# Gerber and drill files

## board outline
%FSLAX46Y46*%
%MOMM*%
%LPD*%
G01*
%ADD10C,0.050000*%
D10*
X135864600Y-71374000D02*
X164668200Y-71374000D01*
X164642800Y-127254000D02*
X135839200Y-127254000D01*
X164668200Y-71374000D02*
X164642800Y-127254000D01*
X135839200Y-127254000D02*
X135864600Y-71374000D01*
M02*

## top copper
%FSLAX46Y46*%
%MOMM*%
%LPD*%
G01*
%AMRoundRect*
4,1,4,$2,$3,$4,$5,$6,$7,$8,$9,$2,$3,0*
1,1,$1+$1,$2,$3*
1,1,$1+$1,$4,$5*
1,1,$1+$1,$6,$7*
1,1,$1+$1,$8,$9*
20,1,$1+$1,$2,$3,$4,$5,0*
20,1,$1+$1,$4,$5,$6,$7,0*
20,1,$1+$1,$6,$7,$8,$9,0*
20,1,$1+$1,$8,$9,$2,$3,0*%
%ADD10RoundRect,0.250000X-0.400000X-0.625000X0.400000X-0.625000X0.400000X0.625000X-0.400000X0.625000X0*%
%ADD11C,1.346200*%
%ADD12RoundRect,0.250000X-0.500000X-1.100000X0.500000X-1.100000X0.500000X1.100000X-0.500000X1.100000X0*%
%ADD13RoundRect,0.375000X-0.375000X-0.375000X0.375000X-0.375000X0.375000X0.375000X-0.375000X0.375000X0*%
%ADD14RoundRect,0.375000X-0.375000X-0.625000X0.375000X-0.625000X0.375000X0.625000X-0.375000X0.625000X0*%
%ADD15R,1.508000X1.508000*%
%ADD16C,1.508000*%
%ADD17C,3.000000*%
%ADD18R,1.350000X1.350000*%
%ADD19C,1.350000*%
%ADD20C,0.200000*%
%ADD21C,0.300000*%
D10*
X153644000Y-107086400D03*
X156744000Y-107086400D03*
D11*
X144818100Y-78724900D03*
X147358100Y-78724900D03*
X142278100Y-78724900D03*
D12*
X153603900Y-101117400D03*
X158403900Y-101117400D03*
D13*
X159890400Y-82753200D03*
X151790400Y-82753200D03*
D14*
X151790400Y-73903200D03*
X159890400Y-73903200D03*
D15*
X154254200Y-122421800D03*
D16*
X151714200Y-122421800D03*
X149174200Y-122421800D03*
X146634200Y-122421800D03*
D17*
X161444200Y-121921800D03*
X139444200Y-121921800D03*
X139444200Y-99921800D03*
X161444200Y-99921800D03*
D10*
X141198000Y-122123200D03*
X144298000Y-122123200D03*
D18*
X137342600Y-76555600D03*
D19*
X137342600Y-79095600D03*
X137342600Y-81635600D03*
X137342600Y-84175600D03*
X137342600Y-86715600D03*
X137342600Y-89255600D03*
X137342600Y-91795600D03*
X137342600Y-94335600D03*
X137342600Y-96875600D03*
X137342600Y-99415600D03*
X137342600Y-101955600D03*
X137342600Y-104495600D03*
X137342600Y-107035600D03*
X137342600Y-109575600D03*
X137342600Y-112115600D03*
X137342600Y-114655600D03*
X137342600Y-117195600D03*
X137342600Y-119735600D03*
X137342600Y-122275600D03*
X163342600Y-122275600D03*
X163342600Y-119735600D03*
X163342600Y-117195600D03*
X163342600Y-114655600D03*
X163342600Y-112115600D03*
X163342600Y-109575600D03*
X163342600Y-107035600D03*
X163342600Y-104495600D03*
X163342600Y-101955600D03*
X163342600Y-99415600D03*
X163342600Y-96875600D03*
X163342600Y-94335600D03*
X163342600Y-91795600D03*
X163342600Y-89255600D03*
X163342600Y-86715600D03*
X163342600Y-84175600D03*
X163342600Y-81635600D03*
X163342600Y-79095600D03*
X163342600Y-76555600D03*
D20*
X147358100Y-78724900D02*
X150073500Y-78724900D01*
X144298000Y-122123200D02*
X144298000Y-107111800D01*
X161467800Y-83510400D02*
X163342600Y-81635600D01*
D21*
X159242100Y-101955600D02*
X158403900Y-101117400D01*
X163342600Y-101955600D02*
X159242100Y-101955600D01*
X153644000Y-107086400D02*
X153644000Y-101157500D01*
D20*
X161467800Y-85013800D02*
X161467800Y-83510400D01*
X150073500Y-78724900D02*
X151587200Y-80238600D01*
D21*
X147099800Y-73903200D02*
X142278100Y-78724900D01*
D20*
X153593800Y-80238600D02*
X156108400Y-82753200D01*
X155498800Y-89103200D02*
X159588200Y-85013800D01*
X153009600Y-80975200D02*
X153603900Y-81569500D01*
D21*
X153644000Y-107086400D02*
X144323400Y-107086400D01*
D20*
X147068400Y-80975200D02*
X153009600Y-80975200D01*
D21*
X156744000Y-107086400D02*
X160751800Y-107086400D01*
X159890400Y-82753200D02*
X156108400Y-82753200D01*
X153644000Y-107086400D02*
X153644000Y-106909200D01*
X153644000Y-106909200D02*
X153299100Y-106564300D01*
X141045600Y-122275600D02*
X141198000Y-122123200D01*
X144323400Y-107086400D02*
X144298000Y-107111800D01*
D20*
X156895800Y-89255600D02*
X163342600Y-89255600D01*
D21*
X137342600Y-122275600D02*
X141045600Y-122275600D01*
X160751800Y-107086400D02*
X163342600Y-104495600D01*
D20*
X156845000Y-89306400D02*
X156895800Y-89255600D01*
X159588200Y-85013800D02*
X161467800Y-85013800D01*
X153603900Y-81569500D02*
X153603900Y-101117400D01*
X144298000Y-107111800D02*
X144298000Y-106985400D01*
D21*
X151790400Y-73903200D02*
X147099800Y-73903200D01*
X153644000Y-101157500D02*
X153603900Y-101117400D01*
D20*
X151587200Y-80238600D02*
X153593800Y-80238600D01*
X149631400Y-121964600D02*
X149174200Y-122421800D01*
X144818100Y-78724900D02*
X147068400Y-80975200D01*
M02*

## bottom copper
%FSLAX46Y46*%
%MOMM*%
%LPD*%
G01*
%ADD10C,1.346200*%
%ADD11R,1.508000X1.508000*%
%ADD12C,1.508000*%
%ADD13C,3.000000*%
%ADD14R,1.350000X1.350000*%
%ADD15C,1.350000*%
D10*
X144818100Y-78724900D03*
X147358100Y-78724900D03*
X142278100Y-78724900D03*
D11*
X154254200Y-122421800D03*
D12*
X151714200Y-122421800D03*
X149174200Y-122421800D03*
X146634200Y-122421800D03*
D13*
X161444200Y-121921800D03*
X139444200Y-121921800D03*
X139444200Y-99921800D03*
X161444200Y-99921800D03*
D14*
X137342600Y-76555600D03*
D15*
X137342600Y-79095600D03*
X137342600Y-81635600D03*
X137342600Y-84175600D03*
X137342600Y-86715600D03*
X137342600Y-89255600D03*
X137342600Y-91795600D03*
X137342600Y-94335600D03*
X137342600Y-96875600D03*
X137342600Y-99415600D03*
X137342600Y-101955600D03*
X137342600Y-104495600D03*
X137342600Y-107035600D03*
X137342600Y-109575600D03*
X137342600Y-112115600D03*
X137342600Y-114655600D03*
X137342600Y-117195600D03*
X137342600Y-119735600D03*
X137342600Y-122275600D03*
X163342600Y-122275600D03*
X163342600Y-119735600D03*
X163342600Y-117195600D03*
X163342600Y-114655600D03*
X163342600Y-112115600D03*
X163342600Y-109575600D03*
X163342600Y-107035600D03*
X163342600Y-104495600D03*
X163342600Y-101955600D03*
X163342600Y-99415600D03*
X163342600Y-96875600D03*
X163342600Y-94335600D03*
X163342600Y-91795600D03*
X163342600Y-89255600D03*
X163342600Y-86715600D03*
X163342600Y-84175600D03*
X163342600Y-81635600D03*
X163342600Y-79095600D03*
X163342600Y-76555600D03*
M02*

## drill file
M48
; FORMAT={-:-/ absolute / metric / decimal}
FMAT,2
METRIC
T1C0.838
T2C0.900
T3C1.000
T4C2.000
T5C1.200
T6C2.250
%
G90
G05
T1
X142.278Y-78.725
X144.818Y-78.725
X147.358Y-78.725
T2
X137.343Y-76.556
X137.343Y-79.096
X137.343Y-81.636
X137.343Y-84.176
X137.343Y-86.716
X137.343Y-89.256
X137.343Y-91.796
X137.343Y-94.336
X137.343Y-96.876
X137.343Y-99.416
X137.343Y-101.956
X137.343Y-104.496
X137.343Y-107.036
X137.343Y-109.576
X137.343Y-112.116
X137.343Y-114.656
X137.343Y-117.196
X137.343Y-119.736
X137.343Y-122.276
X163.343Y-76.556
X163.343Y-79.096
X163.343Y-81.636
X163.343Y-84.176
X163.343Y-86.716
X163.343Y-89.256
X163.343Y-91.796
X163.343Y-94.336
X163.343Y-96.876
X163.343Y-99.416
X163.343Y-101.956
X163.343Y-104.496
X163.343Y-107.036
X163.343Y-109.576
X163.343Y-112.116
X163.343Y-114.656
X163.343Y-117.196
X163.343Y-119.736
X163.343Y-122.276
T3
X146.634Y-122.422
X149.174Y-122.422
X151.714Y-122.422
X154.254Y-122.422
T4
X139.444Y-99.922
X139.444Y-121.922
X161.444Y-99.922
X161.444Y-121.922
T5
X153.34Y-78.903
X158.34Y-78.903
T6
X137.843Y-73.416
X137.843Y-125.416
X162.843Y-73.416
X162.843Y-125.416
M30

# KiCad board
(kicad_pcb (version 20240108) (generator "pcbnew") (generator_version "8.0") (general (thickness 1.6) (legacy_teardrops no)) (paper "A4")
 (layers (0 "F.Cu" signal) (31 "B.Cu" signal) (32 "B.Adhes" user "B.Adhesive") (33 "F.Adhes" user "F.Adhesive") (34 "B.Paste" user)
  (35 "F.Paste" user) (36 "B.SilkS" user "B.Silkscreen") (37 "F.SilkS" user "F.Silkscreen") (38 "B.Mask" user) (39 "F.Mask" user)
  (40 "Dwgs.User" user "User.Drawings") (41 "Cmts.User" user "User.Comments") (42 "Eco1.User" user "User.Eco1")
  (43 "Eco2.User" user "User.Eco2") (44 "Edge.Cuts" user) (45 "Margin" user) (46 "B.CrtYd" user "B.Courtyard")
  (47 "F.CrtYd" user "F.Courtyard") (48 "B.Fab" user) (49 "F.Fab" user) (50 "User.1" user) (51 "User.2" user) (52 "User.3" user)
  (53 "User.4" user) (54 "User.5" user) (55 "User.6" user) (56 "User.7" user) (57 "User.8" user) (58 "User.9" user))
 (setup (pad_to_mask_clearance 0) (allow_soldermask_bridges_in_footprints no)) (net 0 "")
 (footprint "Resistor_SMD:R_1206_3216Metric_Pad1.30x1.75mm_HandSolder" (layer "F.Cu") (at 155.194 107.0864)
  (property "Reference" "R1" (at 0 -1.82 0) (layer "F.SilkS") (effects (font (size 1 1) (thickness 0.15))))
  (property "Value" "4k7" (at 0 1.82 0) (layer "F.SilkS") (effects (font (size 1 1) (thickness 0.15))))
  (pad "1" smd roundrect (at -1.55 0) (size 1.3 1.75) (layers "F.Cu" "F.Paste" "F.Mask") (roundrect_rratio 0.192308))
  (pad "2" smd roundrect (at 1.55 0) (size 1.3 1.75) (layers "F.Cu" "F.Paste" "F.Mask") (roundrect_rratio 0.192308)))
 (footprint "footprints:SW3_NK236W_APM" (layer "F.Cu") (at 144.8181 78.7249 180)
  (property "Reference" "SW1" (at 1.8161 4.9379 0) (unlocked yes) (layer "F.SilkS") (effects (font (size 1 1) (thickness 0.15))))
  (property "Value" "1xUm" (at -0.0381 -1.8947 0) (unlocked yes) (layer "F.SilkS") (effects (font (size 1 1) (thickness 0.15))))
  (pad "1" thru_hole circle (at 0 0 180) (size 1.3462 1.3462) (drill 0.8382) (layers "*.Cu" "*.Mask") (remove_unused_layers no))
  (pad "2" thru_hole circle (at -2.54 0 180) (size 1.3462 1.3462) (drill 0.8382) (layers "*.Cu" "*.Mask") (remove_unused_layers no))
  (pad "3" thru_hole circle (at 2.54 0 180) (size 1.3462 1.3462) (drill 0.8382) (layers "*.Cu" "*.Mask") (remove_unused_layers no)))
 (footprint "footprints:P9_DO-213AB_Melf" (layer "F.Cu") (at 153.6039 101.1174)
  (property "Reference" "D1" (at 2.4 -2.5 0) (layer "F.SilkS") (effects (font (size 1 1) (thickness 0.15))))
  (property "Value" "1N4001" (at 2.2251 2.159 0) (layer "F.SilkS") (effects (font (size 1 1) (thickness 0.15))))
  (pad "1" smd roundrect (at 0 0) (size 1.5 2.7) (layers "F.Cu" "F.Paste" "F.Mask") (roundrect_rratio 0.1666666667))
  (pad "2" smd roundrect (at 4.8 0) (size 1.5 2.7) (layers "F.Cu" "F.Paste" "F.Mask") (roundrect_rratio 0.1666666667)))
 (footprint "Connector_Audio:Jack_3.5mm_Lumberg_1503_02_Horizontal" (layer "F.Cu") (at 155.8404 76.4032)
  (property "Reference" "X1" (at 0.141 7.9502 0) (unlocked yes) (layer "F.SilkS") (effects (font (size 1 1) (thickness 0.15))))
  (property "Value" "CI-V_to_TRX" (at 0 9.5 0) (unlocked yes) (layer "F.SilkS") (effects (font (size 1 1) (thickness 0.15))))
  (pad "" np_thru_hole circle (at -2.5 2.5) (size 1.2 1.2) (drill 1.2) (layers "F&B.Cu" "*.Mask"))
  (pad "" np_thru_hole circle (at 2.5 2.5) (size 1.2 1.2) (drill 1.2) (layers "F&B.Cu" "*.Mask"))
  (pad "R" smd roundrect (at 4.05 6.35) (size 1.5 1.5) (layers "F.Cu" "F.Paste" "F.Mask") (roundrect_rratio 0.25))
  (pad "S" smd roundrect (at -4.05 6.35) (size 1.5 1.5) (layers "F.Cu" "F.Paste" "F.Mask") (roundrect_rratio 0.25))
  (pad "T" smd roundrect (at -4.05 -2.5) (size 1.5 2) (layers "F.Cu" "F.Paste" "F.Mask") (roundrect_rratio 0.25))
  (pad "T" smd roundrect (at 4.05 -2.5) (size 1.5 2) (layers "F.Cu" "F.Paste" "F.Mask") (roundrect_rratio 0.25)))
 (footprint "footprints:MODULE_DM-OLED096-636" (layer "F.Cu") (at 150.4442 110.9218 180)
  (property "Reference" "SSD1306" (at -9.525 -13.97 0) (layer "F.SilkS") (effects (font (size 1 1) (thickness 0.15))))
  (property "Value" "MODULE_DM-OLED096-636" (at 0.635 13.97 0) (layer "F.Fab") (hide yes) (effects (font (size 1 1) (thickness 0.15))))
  (pad "1" thru_hole rect (at -3.81 -11.5 180) (size 1.508 1.508) (drill 1) (layers "*.Cu" "*.Mask") (remove_unused_layers no)
   (solder_mask_margin 0.102))
  (pad "2" thru_hole circle (at -1.27 -11.5 180) (size 1.508 1.508) (drill 1) (layers "*.Cu" "*.Mask") (remove_unused_layers no)
   (solder_mask_margin 0.102))
  (pad "3" thru_hole circle (at 1.27 -11.5 180) (size 1.508 1.508) (drill 1) (layers "*.Cu" "*.Mask") (remove_unused_layers no)
   (solder_mask_margin 0.102))
  (pad "4" thru_hole circle (at 3.81 -11.5 180) (size 1.508 1.508) (drill 1) (layers "*.Cu" "*.Mask") (remove_unused_layers no)
   (solder_mask_margin 0.102))
  (pad "S1" thru_hole circle (at -11 -11 180) (size 3 3) (drill 2) (layers "*.Cu" "*.Mask") (remove_unused_layers no)
   (solder_mask_margin 0.102))
  (pad "S2" thru_hole circle (at 11 -11 180) (size 3 3) (drill 2) (layers "*.Cu" "*.Mask") (remove_unused_layers no)
   (solder_mask_margin 0.102))
  (pad "S3" thru_hole circle (at 11 11 180) (size 3 3) (drill 2) (layers "*.Cu" "*.Mask") (remove_unused_layers no)
   (solder_mask_margin 0.102))
  (pad "S4" thru_hole circle (at -11 11 180) (size 3 3) (drill 2) (layers "*.Cu" "*.Mask") (remove_unused_layers no)
   (solder_mask_margin 0.102)))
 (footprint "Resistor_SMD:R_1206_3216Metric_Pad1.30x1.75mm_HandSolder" (layer "F.Cu") (at 142.748 122.1232)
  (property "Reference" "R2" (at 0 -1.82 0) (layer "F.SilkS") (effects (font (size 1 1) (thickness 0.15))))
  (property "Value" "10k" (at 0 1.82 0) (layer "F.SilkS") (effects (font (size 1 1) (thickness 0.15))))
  (pad "1" smd roundrect (at -1.55 0) (size 1.3 1.75) (layers "F.Cu" "F.Paste" "F.Mask") (roundrect_rratio 0.192308))
  (pad "2" smd roundrect (at 1.55 0) (size 1.3 1.75) (layers "F.Cu" "F.Paste" "F.Mask") (roundrect_rratio 0.192308)))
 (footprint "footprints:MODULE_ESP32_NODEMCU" (layer "B.Cu") (at 150.3426 99.4156 180)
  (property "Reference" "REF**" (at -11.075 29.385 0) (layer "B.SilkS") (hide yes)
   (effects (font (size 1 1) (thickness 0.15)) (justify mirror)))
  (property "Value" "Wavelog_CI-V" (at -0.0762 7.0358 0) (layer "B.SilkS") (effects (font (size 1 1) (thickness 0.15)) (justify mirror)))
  (pad "" np_thru_hole circle (at -12.5 -26 180) (size 2.25 2.25) (drill 2.25) (layers "*.Cu" "*.Mask"))
  (pad "" np_thru_hole circle (at -12.5 26 180) (size 2.25 2.25) (drill 2.25) (layers "*.Cu" "*.Mask"))
  (pad "" np_thru_hole circle (at 12.5 -26 180) (size 2.25 2.25) (drill 2.25) (layers "*.Cu" "*.Mask"))
  (pad "" np_thru_hole circle (at 12.5 26 180) (size 2.25 2.25) (drill 2.25) (layers "*.Cu" "*.Mask"))
  (pad "J4_1" thru_hole rect (at 13 22.86 180) (size 1.35 1.35) (drill 0.9) (layers "*.Cu" "*.Mask") (remove_unused_layers no)
   (solder_mask_margin 0.102))
  (pad "J4_2" thru_hole circle (at 13 20.32 180) (size 1.35 1.35) (drill 0.9) (layers "*.Cu" "*.Mask") (remove_unused_layers no)
   (solder_mask_margin 0.102))
  (pad "J4_3" thru_hole circle (at 13 17.78 180) (size 1.35 1.35) (drill 0.9) (layers "*.Cu" "*.Mask") (remove_unused_layers no)
   (solder_mask_margin 0.102))
  (pad "J4_4" thru_hole circle (at 13 15.24 180) (size 1.35 1.35) (drill 0.9) (layers "*.Cu" "*.Mask") (remove_unused_layers no)
   (solder_mask_margin 0.102))
  (pad "J4_5" thru_hole circle (at 13 12.7 180) (size 1.35 1.35) (drill 0.9) (layers "*.Cu" "*.Mask") (remove_unused_layers no)
   (solder_mask_margin 0.102))
  (pad "J4_6" thru_hole circle (at 13 10.16 180) (size 1.35 1.35) (drill 0.9) (layers "*.Cu" "*.Mask") (remove_unused_layers no)
   (solder_mask_margin 0.102))
  (pad "J4_7" thru_hole circle (at 13 7.62 180) (size 1.35 1.35) (drill 0.9) (layers "*.Cu" "*.Mask") (remove_unused_layers no)
   (solder_mask_margin 0.102))
  (pad "J4_8" thru_hole circle (at 13 5.08 180) (size 1.35 1.35) (drill 0.9) (layers "*.Cu" "*.Mask") (remove_unused_layers no)
   (solder_mask_margin 0.102))
  (pad "J4_9" thru_hole circle (at 13 2.54 180) (size 1.35 1.35) (drill 0.9) (layers "*.Cu" "*.Mask") (remove_unused_layers no)
   (solder_mask_margin 0.102))
  (pad "J4_10" thru_hole circle (at 13 0 180) (size 1.35 1.35) (drill 0.9) (layers "*.Cu" "*.Mask") (remove_unused_layers no)
   (solder_mask_margin 0.102))
  (pad "J4_11" thru_hole circle (at 13 -2.54 180) (size 1.35 1.35) (drill 0.9) (layers "*.Cu" "*.Mask") (remove_unused_layers no)
   (solder_mask_margin 0.102))
  (pad "J4_12" thru_hole circle (at 13 -5.08 180) (size 1.35 1.35) (drill 0.9) (layers "*.Cu" "*.Mask") (remove_unused_layers no)
   (solder_mask_margin 0.102))
  (pad "J4_13" thru_hole circle (at 13 -7.62 180) (size 1.35 1.35) (drill 0.9) (layers "*.Cu" "*.Mask") (remove_unused_layers no)
   (solder_mask_margin 0.102))
  (pad "J4_14" thru_hole circle (at 13 -10.16 180) (size 1.35 1.35) (drill 0.9) (layers "*.Cu" "*.Mask") (remove_unused_layers no)
   (solder_mask_margin 0.102))
  (pad "J4_15" thru_hole circle (at 13 -12.7 180) (size 1.35 1.35) (drill 0.9) (layers "*.Cu" "*.Mask") (remove_unused_layers no)
   (solder_mask_margin 0.102))
  (pad "J4_16" thru_hole circle (at 13 -15.24 180) (size 1.35 1.35) (drill 0.9) (layers "*.Cu" "*.Mask") (remove_unused_layers no)
   (solder_mask_margin 0.102))
  (pad "J4_17" thru_hole circle (at 13 -17.78 180) (size 1.35 1.35) (drill 0.9) (layers "*.Cu" "*.Mask") (remove_unused_layers no)
   (solder_mask_margin 0.102))
  (pad "J4_18" thru_hole circle (at 13 -20.32 180) (size 1.35 1.35) (drill 0.9) (layers "*.Cu" "*.Mask") (remove_unused_layers no)
   (solder_mask_margin 0.102))
  (pad "J4_19" thru_hole circle (at 13 -22.86 180) (size 1.35 1.35) (drill 0.9) (layers "*.Cu" "*.Mask") (remove_unused_layers no)
   (solder_mask_margin 0.102))
  (pad "J5_1" thru_hole circle (at -13 -22.86 180) (size 1.35 1.35) (drill 0.9) (layers "*.Cu" "*.Mask") (remove_unused_layers no)
   (solder_mask_margin 0.102))
  (pad "J5_2" thru_hole circle (at -13 -20.32 180) (size 1.35 1.35) (drill 0.9) (layers "*.Cu" "*.Mask") (remove_unused_layers no)
   (solder_mask_margin 0.102))
  (pad "J5_3" thru_hole circle (at -13 -17.78 180) (size 1.35 1.35) (drill 0.9) (layers "*.Cu" "*.Mask") (remove_unused_layers no)
   (solder_mask_margin 0.102))
  (pad "J5_4" thru_hole circle (at -13 -15.24 180) (size 1.35 1.35) (drill 0.9) (layers "*.Cu" "*.Mask") (remove_unused_layers no)
   (solder_mask_margin 0.102))
  (pad "J5_5" thru_hole circle (at -13 -12.7 180) (size 1.35 1.35) (drill 0.9) (layers "*.Cu" "*.Mask") (remove_unused_layers no)
   (solder_mask_margin 0.102))
  (pad "J5_6" thru_hole circle (at -13 -10.16 180) (size 1.35 1.35) (drill 0.9) (layers "*.Cu" "*.Mask") (remove_unused_layers no)
   (solder_mask_margin 0.102))
  (pad "J5_7" thru_hole circle (at -13 -7.62 180) (size 1.35 1.35) (drill 0.9) (layers "*.Cu" "*.Mask") (remove_unused_layers no)
   (solder_mask_margin 0.102))
  (pad "J5_8" thru_hole circle (at -13 -5.08 180) (size 1.35 1.35) (drill 0.9) (layers "*.Cu" "*.Mask") (remove_unused_layers no)
   (solder_mask_margin 0.102))
  (pad "J5_9" thru_hole circle (at -13 -2.54 180) (size 1.35 1.35) (drill 0.9) (layers "*.Cu" "*.Mask") (remove_unused_layers no)
   (solder_mask_margin 0.102))
  (pad "J5_10" thru_hole circle (at -13 0 180) (size 1.35 1.35) (drill 0.9) (layers "*.Cu" "*.Mask") (remove_unused_layers no)
   (solder_mask_margin 0.102))
  (pad "J5_11" thru_hole circle (at -13 2.54 180) (size 1.35 1.35) (drill 0.9) (layers "*.Cu" "*.Mask") (remove_unused_layers no)
   (solder_mask_margin 0.102))
  (pad "J5_12" thru_hole circle (at -13 5.08 180) (size 1.35 1.35) (drill 0.9) (layers "*.Cu" "*.Mask") (remove_unused_layers no)
   (solder_mask_margin 0.102))
  (pad "J5_13" thru_hole circle (at -13 7.62 180) (size 1.35 1.35) (drill 0.9) (layers "*.Cu" "*.Mask") (remove_unused_layers no)
   (solder_mask_margin 0.102))
  (pad "J5_14" thru_hole circle (at -13 10.16 180) (size 1.35 1.35) (drill 0.9) (layers "*.Cu" "*.Mask") (remove_unused_layers no)
   (solder_mask_margin 0.102))
  (pad "J5_15" thru_hole circle (at -13 12.7 180) (size 1.35 1.35) (drill 0.9) (layers "*.Cu" "*.Mask") (remove_unused_layers no)
   (solder_mask_margin 0.102))
  (pad "J5_16" thru_hole circle (at -13 15.24 180) (size 1.35 1.35) (drill 0.9) (layers "*.Cu" "*.Mask") (remove_unused_layers no)
   (solder_mask_margin 0.102))
  (pad "J5_17" thru_hole circle (at -13 17.78 180) (size 1.35 1.35) (drill 0.9) (layers "*.Cu" "*.Mask") (remove_unused_layers no)
   (solder_mask_margin 0.102))
  (pad "J5_18" thru_hole circle (at -13 20.32 180) (size 1.35 1.35) (drill 0.9) (layers "*.Cu" "*.Mask") (remove_unused_layers no)
   (solder_mask_margin 0.102))
  (pad "J5_19" thru_hole circle (at -13 22.86 180) (size 1.35 1.35) (drill 0.9) (layers "*.Cu" "*.Mask") (remove_unused_layers no)
   (solder_mask_margin 0.102)))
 (gr_line (start 135.8646 71.374) (end 164.6682 71.374) (stroke (width 0.05) (type default)) (layer "Edge.Cuts"))
 (gr_line (start 164.6428 127.254) (end 135.8392 127.254) (stroke (width 0.05) (type default)) (layer "Edge.Cuts"))
 (gr_line (start 164.6682 71.374) (end 164.6428 127.254) (stroke (width 0.05) (type default)) (layer "Edge.Cuts"))
 (gr_line (start 135.8392 127.254) (end 135.8646 71.374) (stroke (width 0.05) (type default)) (layer "Edge.Cuts"))
 (segment (start 147.3581 78.7249) (end 150.0735 78.7249) (width 0.2) (layer "F.Cu") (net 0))
 (segment (start 144.298 122.1232) (end 144.298 107.1118) (width 0.2) (layer "F.Cu") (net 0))
 (segment (start 161.4678 83.5104) (end 163.3426 81.6356) (width 0.2) (layer "F.Cu") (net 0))
 (segment (start 159.2421 101.9556) (end 158.4039 101.1174) (width 0.3) (layer "F.Cu") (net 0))
 (segment (start 163.3426 101.9556) (end 159.2421 101.9556) (width 0.3) (layer "F.Cu") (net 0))
 (segment (start 153.644 107.0864) (end 153.644 101.1575) (width 0.3) (layer "F.Cu") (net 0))
 (segment (start 161.4678 85.0138) (end 161.4678 83.5104) (width 0.2) (layer "F.Cu") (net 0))
 (segment (start 150.0735 78.7249) (end 151.5872 80.2386) (width 0.2) (layer "F.Cu") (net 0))
 (segment (start 147.0998 73.9032) (end 142.2781 78.7249) (width 0.3) (layer "F.Cu") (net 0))
 (segment (start 153.5938 80.2386) (end 156.1084 82.7532) (width 0.2) (layer "F.Cu") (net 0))
 (segment (start 155.4988 89.1032) (end 159.5882 85.0138) (width 0.2) (layer "F.Cu") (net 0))
 (segment (start 153.0096 80.9752) (end 153.6039 81.5695) (width 0.2) (layer "F.Cu") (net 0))
 (segment (start 153.644 107.0864) (end 144.3234 107.0864) (width 0.3) (layer "F.Cu") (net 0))
 (segment (start 147.0684 80.9752) (end 153.0096 80.9752) (width 0.2) (layer "F.Cu") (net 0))
 (segment (start 156.744 107.0864) (end 160.7518 107.0864) (width 0.3) (layer "F.Cu") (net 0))
 (segment (start 159.8904 82.7532) (end 156.1084 82.7532) (width 0.3) (layer "F.Cu") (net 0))
 (segment (start 153.644 107.0864) (end 153.644 106.9092) (width 0.3) (layer "F.Cu") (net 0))
 (segment (start 153.644 106.9092) (end 153.2991 106.5643) (width 0.3) (layer "F.Cu") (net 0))
 (segment (start 141.0456 122.2756) (end 141.198 122.1232) (width 0.3) (layer "F.Cu") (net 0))
 (segment (start 144.3234 107.0864) (end 144.298 107.1118) (width 0.3) (layer "F.Cu") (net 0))
 (segment (start 156.8958 89.2556) (end 163.3426 89.2556) (width 0.2) (layer "F.Cu") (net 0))
 (segment (start 137.3426 122.2756) (end 141.0456 122.2756) (width 0.3) (layer "F.Cu") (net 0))
 (segment (start 160.7518 107.0864) (end 163.3426 104.4956) (width 0.3) (layer "F.Cu") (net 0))
 (segment (start 156.845 89.3064) (end 156.8958 89.2556) (width 0.2) (layer "F.Cu") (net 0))
 (segment (start 159.5882 85.0138) (end 161.4678 85.0138) (width 0.2) (layer "F.Cu") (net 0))
 (segment (start 153.6039 81.5695) (end 153.6039 101.1174) (width 0.2) (layer "F.Cu") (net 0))
 (segment (start 144.298 107.1118) (end 144.298 106.9854) (width 0.2) (layer "F.Cu") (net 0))
 (segment (start 151.7904 73.9032) (end 147.0998 73.9032) (width 0.3) (layer "F.Cu") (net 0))
 (segment (start 153.644 101.1575) (end 153.6039 101.1174) (width 0.3) (layer "F.Cu") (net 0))
 (segment (start 151.5872 80.2386) (end 153.5938 80.2386) (width 0.2) (layer "F.Cu") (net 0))
 (segment (start 149.6314 121.9646) (end 149.1742 122.4218) (width 0.2) (layer "F.Cu") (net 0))
 (segment (start 144.8181 78.7249) (end 147.0684 80.9752) (width 0.2) (layer "F.Cu") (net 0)))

